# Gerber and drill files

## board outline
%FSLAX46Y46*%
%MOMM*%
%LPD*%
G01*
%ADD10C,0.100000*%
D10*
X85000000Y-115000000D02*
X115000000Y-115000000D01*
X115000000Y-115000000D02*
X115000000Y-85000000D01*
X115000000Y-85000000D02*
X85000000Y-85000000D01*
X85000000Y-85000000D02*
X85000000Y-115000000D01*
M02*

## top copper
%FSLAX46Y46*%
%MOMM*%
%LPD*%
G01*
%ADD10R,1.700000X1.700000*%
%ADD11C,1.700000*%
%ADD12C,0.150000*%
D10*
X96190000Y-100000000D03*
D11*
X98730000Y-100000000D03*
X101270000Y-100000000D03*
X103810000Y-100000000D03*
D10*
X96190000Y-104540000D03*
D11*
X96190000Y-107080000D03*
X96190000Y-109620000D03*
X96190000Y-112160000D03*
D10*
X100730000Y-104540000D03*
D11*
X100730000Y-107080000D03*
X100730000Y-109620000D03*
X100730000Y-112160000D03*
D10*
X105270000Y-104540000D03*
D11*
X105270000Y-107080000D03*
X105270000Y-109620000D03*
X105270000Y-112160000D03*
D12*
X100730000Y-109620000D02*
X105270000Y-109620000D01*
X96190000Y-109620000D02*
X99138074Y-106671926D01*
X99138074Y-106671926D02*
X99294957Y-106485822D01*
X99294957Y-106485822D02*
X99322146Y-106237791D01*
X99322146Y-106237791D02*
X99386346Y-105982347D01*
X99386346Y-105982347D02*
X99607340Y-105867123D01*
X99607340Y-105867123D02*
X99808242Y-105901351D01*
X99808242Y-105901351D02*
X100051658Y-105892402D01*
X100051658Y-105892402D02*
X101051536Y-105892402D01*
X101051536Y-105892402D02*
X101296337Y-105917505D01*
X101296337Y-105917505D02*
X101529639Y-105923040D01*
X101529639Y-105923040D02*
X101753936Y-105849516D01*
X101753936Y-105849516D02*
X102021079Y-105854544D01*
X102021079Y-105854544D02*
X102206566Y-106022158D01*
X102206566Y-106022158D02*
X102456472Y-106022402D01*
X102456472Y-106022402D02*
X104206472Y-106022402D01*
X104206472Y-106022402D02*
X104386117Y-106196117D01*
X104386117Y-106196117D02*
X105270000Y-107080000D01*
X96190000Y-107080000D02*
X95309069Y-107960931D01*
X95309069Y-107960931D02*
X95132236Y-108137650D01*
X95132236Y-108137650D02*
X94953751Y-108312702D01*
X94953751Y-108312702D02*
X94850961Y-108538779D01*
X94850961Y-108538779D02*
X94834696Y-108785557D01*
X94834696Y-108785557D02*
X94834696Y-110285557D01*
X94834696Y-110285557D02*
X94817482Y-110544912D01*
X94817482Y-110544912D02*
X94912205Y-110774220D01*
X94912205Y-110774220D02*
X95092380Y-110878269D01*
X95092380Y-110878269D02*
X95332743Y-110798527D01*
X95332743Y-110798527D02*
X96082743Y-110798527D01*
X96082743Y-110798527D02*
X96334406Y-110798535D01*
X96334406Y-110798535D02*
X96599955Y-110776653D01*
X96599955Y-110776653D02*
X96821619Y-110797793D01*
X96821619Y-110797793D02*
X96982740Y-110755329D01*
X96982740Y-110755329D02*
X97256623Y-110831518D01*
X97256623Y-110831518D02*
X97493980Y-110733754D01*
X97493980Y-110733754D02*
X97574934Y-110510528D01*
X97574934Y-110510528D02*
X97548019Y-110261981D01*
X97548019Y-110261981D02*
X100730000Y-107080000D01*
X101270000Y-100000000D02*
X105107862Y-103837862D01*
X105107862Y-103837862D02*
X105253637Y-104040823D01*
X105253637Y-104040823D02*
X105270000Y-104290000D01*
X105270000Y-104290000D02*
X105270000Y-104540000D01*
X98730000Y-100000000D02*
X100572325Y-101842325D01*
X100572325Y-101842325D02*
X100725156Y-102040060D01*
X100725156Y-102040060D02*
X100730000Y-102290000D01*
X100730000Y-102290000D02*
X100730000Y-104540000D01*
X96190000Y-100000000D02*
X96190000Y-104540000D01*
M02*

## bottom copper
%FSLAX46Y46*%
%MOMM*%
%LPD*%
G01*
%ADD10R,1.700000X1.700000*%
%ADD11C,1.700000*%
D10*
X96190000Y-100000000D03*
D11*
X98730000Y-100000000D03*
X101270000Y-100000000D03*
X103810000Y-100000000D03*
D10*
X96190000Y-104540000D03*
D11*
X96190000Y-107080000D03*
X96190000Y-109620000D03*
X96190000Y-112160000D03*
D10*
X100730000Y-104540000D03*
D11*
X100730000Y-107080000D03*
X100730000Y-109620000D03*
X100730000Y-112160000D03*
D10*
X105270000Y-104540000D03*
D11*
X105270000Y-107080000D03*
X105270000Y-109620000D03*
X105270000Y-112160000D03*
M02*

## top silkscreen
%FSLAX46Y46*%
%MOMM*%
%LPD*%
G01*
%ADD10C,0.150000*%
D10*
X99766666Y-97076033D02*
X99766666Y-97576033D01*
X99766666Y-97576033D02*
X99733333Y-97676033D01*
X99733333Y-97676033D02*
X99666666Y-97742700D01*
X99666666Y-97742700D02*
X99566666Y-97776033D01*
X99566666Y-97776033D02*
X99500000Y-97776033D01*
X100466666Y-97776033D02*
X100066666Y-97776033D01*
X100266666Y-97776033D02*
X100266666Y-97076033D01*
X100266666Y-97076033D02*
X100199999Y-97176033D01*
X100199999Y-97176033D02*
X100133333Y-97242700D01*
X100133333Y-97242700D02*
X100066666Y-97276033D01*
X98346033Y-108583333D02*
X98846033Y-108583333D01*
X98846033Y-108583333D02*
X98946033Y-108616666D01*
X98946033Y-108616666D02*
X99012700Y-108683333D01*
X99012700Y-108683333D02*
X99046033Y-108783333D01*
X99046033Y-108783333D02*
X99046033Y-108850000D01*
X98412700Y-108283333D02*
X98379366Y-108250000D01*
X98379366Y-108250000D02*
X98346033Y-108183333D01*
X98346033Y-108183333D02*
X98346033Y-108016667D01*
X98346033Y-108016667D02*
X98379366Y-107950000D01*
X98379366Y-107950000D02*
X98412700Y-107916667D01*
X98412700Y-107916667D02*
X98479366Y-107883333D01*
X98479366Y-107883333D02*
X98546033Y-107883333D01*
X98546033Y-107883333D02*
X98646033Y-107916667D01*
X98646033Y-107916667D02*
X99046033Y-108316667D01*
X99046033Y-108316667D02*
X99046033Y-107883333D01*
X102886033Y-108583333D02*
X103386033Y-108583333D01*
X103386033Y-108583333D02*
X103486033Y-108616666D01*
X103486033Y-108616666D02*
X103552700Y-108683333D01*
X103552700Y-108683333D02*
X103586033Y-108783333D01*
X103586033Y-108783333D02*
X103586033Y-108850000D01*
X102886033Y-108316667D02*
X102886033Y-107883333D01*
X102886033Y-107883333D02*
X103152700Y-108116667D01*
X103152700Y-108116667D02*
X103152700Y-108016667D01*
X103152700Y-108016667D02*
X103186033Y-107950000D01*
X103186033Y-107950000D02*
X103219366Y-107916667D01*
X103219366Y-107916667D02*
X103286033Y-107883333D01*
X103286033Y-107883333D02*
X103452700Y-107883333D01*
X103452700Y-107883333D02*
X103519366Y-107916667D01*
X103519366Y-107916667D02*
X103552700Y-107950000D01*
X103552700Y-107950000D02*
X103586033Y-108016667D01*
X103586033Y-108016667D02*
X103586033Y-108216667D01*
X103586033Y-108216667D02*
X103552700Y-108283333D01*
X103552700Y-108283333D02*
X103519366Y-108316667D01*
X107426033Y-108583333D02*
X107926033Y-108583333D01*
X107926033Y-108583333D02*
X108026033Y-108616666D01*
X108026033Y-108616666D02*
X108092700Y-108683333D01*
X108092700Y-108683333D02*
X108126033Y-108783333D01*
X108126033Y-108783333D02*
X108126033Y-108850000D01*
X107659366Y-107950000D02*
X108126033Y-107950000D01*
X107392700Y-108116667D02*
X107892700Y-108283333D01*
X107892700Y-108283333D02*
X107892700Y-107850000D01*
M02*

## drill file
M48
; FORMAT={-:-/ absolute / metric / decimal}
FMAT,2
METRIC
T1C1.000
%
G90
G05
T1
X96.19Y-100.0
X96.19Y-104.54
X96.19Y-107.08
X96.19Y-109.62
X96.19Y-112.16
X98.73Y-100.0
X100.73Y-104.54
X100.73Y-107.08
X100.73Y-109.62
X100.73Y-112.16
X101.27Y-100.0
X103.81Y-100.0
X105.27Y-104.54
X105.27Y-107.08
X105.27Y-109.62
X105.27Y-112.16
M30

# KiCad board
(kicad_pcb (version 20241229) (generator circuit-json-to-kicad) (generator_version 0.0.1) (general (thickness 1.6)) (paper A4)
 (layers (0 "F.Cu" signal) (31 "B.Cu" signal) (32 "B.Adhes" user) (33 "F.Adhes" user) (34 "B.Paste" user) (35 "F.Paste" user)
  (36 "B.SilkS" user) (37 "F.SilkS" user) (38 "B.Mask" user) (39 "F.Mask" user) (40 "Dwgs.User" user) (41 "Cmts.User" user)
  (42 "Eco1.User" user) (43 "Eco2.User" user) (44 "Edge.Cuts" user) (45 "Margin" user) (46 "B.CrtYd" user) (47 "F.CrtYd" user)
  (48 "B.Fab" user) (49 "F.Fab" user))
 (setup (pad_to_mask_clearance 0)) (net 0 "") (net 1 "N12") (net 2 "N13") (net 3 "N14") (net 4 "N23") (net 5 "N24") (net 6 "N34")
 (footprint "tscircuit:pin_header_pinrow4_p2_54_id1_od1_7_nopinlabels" (layer F.Cu) (at 100 100 0)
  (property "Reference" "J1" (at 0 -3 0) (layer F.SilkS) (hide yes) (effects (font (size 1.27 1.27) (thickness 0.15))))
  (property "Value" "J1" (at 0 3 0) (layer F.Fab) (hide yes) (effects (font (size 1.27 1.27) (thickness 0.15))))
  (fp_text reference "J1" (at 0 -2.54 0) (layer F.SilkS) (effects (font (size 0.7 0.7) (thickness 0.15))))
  (pad "1" thru_hole rect (at -3.81 0 0) (size 1.7 1.7) (drill 1) (layers *.Cu *.Mask) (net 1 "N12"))
  (pad "2" thru_hole circle (at -1.27 0 0) (size 1.7 1.7) (drill 1) (layers *.Cu *.Mask) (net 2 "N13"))
  (pad "3" thru_hole circle (at 1.27 0 0) (size 1.7 1.7) (drill 1) (layers *.Cu *.Mask) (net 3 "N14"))
  (pad "4" thru_hole circle (at 3.81 0 0) (size 1.7 1.7) (drill 1) (layers *.Cu *.Mask)))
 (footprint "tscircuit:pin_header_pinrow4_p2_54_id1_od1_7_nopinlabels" (layer F.Cu) (at 96.19 108.35 -90.00000000000001)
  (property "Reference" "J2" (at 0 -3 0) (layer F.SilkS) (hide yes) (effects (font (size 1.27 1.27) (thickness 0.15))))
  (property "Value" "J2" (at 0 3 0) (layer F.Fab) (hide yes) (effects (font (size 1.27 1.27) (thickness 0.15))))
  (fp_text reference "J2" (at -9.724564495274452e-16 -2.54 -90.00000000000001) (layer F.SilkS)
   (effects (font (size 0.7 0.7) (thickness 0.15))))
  (pad "1" thru_hole rect (at -3.8100000000000005 5.705062545910426e-16 270) (size 1.7 1.7) (drill 1) (layers *.Cu *.Mask) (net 1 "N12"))
  (pad "2" thru_hole circle (at -1.2699999999999996 4.2139014913659776e-17 0) (size 1.7 1.7) (drill 1) (layers *.Cu *.Mask) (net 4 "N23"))
  (pad "3" thru_hole circle (at 1.2699999999999996 -4.2139014913659776e-17 0) (size 1.7 1.7) (drill 1) (layers *.Cu *.Mask) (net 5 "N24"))
  (pad "4" thru_hole circle (at 3.8100000000000005 -5.705062545910426e-16 0) (size 1.7 1.7) (drill 1) (layers *.Cu *.Mask)))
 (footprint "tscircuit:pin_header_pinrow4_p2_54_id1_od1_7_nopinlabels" (layer F.Cu) (at 100.73 108.35000000000001 -90.00000000000001)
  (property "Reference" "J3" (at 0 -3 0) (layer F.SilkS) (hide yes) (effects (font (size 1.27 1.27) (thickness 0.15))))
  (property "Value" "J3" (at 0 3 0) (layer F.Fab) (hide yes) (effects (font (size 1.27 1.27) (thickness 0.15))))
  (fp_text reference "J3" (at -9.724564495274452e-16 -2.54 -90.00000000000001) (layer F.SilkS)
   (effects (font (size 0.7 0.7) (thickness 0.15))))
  (pad "1" thru_hole rect (at -3.8100000000000005 7.925508595160739e-16 270) (size 1.7 1.7) (drill 1) (layers *.Cu *.Mask) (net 2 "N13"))
  (pad "2" thru_hole circle (at -1.2699999999999996 2.641836198386911e-16 0) (size 1.7 1.7) (drill 1) (layers *.Cu *.Mask) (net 4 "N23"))
  (pad "3" thru_hole circle (at 1.2699999999999996 -2.641836198386911e-16 0) (size 1.7 1.7) (drill 1) (layers *.Cu *.Mask) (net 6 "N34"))
  (pad "4" thru_hole circle (at 3.8100000000000005 -7.925508595160739e-16 0) (size 1.7 1.7) (drill 1) (layers *.Cu *.Mask)))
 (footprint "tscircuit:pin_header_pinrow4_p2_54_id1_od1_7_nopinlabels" (layer F.Cu)
  (at 105.27000000000001 108.35000000000001 -90.00000000000001)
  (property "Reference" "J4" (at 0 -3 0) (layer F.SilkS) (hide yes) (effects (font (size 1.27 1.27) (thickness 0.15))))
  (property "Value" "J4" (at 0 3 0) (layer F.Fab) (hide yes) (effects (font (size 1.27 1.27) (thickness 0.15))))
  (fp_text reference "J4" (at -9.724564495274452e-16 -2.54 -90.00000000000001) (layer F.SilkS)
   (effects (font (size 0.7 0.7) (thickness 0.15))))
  (pad "1" thru_hole rect (at -3.8100000000000005 5.705062545910426e-16 270) (size 1.7 1.7) (drill 1) (layers *.Cu *.Mask) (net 3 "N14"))
  (pad "2" thru_hole circle (at -1.2699999999999996 4.862282247637224e-16 0) (size 1.7 1.7) (drill 1) (layers *.Cu *.Mask) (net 5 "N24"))
  (pad "3" thru_hole circle (at 1.2699999999999996 -4.862282247637224e-16 0) (size 1.7 1.7) (drill 1) (layers *.Cu *.Mask) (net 6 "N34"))
  (pad "4" thru_hole circle (at 3.8100000000000005 -5.705062545910426e-16 0) (size 1.7 1.7) (drill 1) (layers *.Cu *.Mask)))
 (segment (start 100.73 109.62) (end 105.27000000000001 109.62) (width 0.15) (layer F.Cu) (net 6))
 (segment (start 96.19 109.62) (end 99.13807401949714 106.67192598050286) (width 0.15) (layer F.Cu) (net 5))
 (segment (start 99.13807401949714 106.67192598050286) (end 99.2949574117885 106.48582224405315) (width 0.15) (layer F.Cu) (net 5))
 (segment (start 99.2949574117885 106.48582224405315) (end 99.32214603470558 106.23779128025606) (width 0.15) (layer F.Cu) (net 5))
 (segment (start 99.32214603470558 106.23779128025606) (end 99.38634622607654 105.98234683483743) (width 0.15) (layer F.Cu) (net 5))
 (segment (start 99.38634622607654 105.98234683483743) (end 99.60733992339257 105.86712316196164) (width 0.15) (layer F.Cu) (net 5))
 (segment (start 99.60733992339257 105.86712316196164) (end 99.80824191390279 105.90135081123873) (width 0.15) (layer F.Cu) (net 5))
 (segment (start 99.80824191390279 105.90135081123873) (end 100.05165787031913 105.89240161025909) (width 0.15) (layer F.Cu) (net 5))
 (segment (start 100.05165787031913 105.89240161025909) (end 101.05153608915805 105.89240156788578) (width 0.15) (layer F.Cu) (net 5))
 (segment (start 101.05153608915805 105.89240156788578) (end 101.29633662362976 105.91750478680689) (width 0.15) (layer F.Cu) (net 5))
 (segment (start 101.29633662362976 105.91750478680689) (end 101.52963912367376 105.92303995946095) (width 0.15) (layer F.Cu) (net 5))
 (segment (start 101.52963912367376 105.92303995946095) (end 101.7539364417838 105.84951638923202) (width 0.15) (layer F.Cu) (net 5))
 (segment (start 101.7539364417838 105.84951638923202) (end 102.02107926650245 105.85454352610085) (width 0.15) (layer F.Cu) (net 5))
 (segment (start 102.02107926650245 105.85454352610085) (end 102.20656577039956 106.02215843257409) (width 0.15) (layer F.Cu) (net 5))
 (segment (start 102.20656577039956 106.02215843257409) (end 102.45647217345783 106.02240161025908) (width 0.15) (layer F.Cu) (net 5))
 (segment (start 102.45647217345783 106.02240161025908) (end 104.20647217345783 106.02240161025908) (width 0.15) (layer F.Cu) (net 5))
 (segment (start 104.20647217345783 106.02240161025908) (end 104.38611652351682 106.19611652351682) (width 0.15) (layer F.Cu) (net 5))
 (segment (start 104.38611652351682 106.19611652351682) (end 105.27000000000001 107.08000000000001) (width 0.15) (layer F.Cu) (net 5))
 (segment (start 96.19 107.08) (end 95.30906949419422 107.96093050580578) (width 0.15) (layer F.Cu) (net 4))
 (segment (start 95.30906949419422 107.96093050580578) (end 95.13223591999272 108.13764976729482) (width 0.15) (layer F.Cu) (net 4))
 (segment (start 95.13223591999272 108.13764976729482) (end 94.95375135859925 108.31270193478832) (width 0.15) (layer F.Cu) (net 4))
 (segment (start 94.95375135859925 108.31270193478832) (end 94.85096111185794 108.5387790866457) (width 0.15) (layer F.Cu) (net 4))
 (segment (start 94.85096111185794 108.5387790866457) (end 94.83469646767949 108.78555697905891) (width 0.15) (layer F.Cu) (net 4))
 (segment (start 94.83469646767949 108.78555697905891) (end 94.83469646767949 110.28555697905891) (width 0.15) (layer F.Cu) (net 4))
 (segment (start 94.83469646767949 110.28555697905891) (end 94.81748205589265 110.54491192545305) (width 0.15) (layer F.Cu) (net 4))
 (segment (start 94.81748205589265 110.54491192545305) (end 94.91220527664319 110.77421984879163) (width 0.15) (layer F.Cu) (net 4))
 (segment (start 94.91220527664319 110.77421984879163) (end 95.09238049558903 110.87826901452028) (width 0.15) (layer F.Cu) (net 4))
 (segment (start 95.09238049558903 110.87826901452028) (end 95.33274336535685 110.79852682852155) (width 0.15) (layer F.Cu) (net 4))
 (segment (start 95.33274336535685 110.79852682852155) (end 96.08274336535685 110.79852682852155) (width 0.15) (layer F.Cu) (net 4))
 (segment (start 96.08274336535685 110.79852682852155) (end 96.33440632433276 110.7985347299358) (width 0.15) (layer F.Cu) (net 4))
 (segment (start 96.33440632433276 110.7985347299358) (end 96.5999550091064 110.7766531299792) (width 0.15) (layer F.Cu) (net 4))
 (segment (start 96.5999550091064 110.7766531299792) (end 96.82161906338449 110.79779311663782) (width 0.15) (layer F.Cu) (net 4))
 (segment (start 96.82161906338449 110.79779311663782) (end 96.98273963886854 110.75532936625248) (width 0.15) (layer F.Cu) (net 4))
 (segment (start 96.98273963886854 110.75532936625248) (end 97.25662281889468 110.8315178778145) (width 0.15) (layer F.Cu) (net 4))
 (segment (start 97.25662281889468 110.8315178778145) (end 97.49398027472799 110.73375418241669) (width 0.15) (layer F.Cu) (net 4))
 (segment (start 97.49398027472799 110.73375418241669) (end 97.57493360810754 110.51052755305885) (width 0.15) (layer F.Cu) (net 4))
 (segment (start 97.57493360810754 110.51052755305885) (end 97.54801948466053 110.26198051533947) (width 0.15) (layer F.Cu) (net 4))
 (segment (start 97.54801948466053 110.26198051533947) (end 100.73 107.08) (width 0.15) (layer F.Cu) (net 4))
 (segment (start 101.27 100) (end 105.10786241158964 103.83786241158963) (width 0.15) (layer F.Cu) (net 3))
 (segment (start 105.10786241158964 103.83786241158963) (end 105.25363676561919 104.04082277575598) (width 0.15) (layer F.Cu) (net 3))
 (segment (start 105.25363676561919 104.04082277575598) (end 105.27000000000001 104.29) (width 0.15) (layer F.Cu) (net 3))
 (segment (start 105.27000000000001 104.29) (end 105.27000000000001 104.54) (width 0.15) (layer F.Cu) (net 3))
 (segment (start 98.73 100) (end 100.5723245135854 101.84232451358541) (width 0.15) (layer F.Cu) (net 2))
 (segment (start 100.5723245135854 101.84232451358541) (end 100.72515557761582 102.04006036977569) (width 0.15) (layer F.Cu) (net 2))
 (segment (start 100.72515557761582 102.04006036977569) (end 100.73 102.29) (width 0.15) (layer F.Cu) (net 2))
 (segment (start 100.73 102.29) (end 100.73 104.54) (width 0.15) (layer F.Cu) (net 2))
 (segment (start 96.19 100) (end 96.19 104.53999999999999) (width 0.15) (layer F.Cu) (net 1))
 (gr_line (start 85 115) (end 115 115) (width 0.1) (layer Edge.Cuts))
 (gr_line (start 115 115) (end 115 85) (width 0.1) (layer Edge.Cuts))
 (gr_line (start 115 85) (end 85 85) (width 0.1) (layer Edge.Cuts))
 (gr_line (start 85 85) (end 85 115) (width 0.1) (layer Edge.Cuts)))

